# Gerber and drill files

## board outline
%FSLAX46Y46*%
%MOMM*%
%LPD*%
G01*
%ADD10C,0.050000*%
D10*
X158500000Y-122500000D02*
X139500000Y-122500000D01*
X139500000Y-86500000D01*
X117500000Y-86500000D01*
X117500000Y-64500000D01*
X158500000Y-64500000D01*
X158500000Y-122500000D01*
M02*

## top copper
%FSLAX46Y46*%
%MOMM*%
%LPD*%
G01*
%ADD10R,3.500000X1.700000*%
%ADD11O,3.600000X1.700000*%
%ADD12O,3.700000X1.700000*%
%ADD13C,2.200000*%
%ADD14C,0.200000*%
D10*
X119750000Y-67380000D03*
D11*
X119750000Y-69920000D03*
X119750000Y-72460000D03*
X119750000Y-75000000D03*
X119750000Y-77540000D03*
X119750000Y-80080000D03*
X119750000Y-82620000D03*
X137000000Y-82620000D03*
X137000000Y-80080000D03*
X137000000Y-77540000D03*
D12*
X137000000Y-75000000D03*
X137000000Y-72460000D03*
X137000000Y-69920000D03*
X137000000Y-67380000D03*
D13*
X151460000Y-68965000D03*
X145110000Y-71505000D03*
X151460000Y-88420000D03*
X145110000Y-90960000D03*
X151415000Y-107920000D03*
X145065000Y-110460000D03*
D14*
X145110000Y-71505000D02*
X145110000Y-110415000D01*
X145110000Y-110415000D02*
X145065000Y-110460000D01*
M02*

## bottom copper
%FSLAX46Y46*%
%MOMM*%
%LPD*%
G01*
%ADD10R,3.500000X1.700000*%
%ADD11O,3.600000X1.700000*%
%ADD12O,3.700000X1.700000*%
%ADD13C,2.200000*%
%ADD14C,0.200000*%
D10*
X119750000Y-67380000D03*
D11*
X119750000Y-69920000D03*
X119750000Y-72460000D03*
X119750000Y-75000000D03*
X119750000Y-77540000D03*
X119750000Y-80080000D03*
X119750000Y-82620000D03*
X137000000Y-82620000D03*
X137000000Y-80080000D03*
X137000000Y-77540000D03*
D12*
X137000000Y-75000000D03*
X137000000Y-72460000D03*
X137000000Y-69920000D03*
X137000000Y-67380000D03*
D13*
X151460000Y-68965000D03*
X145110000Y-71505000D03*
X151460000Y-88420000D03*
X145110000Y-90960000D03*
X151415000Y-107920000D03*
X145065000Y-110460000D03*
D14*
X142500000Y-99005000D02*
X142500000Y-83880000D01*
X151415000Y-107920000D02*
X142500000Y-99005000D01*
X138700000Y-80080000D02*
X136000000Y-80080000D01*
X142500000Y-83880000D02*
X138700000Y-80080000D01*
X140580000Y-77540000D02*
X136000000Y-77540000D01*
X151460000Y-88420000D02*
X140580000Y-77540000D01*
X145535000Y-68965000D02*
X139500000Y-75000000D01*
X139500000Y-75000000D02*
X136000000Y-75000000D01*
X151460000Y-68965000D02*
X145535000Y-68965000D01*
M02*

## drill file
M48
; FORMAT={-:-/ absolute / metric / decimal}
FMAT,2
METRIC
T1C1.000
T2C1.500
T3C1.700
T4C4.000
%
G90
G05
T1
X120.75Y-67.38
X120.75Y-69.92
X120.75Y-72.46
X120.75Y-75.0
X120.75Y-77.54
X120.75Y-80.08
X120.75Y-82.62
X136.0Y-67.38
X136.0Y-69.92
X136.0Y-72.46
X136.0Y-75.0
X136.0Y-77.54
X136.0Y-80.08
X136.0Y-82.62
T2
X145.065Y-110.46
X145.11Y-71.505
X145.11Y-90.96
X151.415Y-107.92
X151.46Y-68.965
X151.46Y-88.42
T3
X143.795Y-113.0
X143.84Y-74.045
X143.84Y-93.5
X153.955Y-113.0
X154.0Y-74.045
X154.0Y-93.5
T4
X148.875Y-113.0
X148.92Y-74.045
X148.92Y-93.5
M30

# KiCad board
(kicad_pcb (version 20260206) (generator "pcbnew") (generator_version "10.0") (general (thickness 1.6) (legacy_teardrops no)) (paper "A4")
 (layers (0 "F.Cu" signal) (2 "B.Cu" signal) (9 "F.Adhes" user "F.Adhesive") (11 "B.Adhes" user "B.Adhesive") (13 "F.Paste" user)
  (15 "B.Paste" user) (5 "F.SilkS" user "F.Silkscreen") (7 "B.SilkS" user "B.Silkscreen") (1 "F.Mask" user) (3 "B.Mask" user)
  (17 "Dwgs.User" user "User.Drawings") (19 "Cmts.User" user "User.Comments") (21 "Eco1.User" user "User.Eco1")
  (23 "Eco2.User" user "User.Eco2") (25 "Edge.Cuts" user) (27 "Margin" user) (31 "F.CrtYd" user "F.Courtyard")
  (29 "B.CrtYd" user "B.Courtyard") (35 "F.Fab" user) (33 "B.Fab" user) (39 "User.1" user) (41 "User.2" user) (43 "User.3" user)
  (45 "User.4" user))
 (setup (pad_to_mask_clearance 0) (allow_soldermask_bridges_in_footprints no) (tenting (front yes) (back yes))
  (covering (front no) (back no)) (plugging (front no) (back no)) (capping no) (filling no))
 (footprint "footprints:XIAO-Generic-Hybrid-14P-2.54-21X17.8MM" (layer "F.Cu") (at 128.375 75)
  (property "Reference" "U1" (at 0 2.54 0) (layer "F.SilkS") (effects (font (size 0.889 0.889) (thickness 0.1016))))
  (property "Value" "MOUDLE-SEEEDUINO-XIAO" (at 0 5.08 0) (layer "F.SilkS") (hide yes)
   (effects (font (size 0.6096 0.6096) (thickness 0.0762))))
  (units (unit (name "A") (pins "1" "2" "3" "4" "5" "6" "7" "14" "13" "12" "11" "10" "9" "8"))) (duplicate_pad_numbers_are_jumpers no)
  (pad "1" thru_hole rect (at -7.625 -7.62) (size 3.5 1.7) (drill 1 (offset -1 0)) (layers "*.Cu" "*.Mask") (remove_unused_layers no)
   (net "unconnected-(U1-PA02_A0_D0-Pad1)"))
  (pad "2" thru_hole oval (at -7.625 -5.08) (size 3.6 1.7) (drill 1 (offset -1 0)) (layers "*.Cu" "*.Mask") (remove_unused_layers no)
   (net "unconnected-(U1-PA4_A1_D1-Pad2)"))
  (pad "3" thru_hole oval (at -7.625 -2.54) (size 3.6 1.7) (drill 1 (offset -1 0)) (layers "*.Cu" "*.Mask") (remove_unused_layers no)
   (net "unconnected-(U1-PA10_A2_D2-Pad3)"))
  (pad "4" thru_hole oval (at -7.625 0) (size 3.6 1.7) (drill 1 (offset -1 0)) (layers "*.Cu" "*.Mask") (remove_unused_layers no)
   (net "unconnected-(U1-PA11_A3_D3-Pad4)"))
  (pad "5" thru_hole oval (at -7.625 2.54) (size 3.6 1.7) (drill 1 (offset -1 0)) (layers "*.Cu" "*.Mask") (remove_unused_layers no)
   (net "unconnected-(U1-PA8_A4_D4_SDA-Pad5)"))
  (pad "6" thru_hole oval (at -7.625 5.08 180) (size 3.6 1.7) (drill 1 (offset 1 0)) (layers "*.Cu" "*.Mask") (remove_unused_layers no)
   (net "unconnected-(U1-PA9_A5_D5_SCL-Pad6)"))
  (pad "7" thru_hole oval (at -7.625 7.62) (size 3.6 1.7) (drill 1 (offset -1 0)) (layers "*.Cu" "*.Mask") (remove_unused_layers no)
   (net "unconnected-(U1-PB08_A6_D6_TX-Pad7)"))
  (pad "8" thru_hole oval (at 7.625 7.62) (size 3.6 1.7) (drill 1 (offset 1 0)) (layers "*.Cu" "*.Mask") (remove_unused_layers no)
   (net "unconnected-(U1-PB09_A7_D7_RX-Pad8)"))
  (pad "9" thru_hole oval (at 7.625 5.08) (size 3.6 1.7) (drill 1 (offset 1 0)) (layers "*.Cu" "*.Mask") (remove_unused_layers no)
   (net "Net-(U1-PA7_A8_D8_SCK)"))
  (pad "10" thru_hole oval (at 7.625 2.54) (size 3.6 1.7) (drill 1 (offset 1 0)) (layers "*.Cu" "*.Mask") (remove_unused_layers no)
   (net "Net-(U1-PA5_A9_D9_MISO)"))
  (pad "11" thru_hole oval (at 7.625 0) (size 3.7 1.7) (drill 1 (offset 1 0)) (layers "*.Cu" "*.Mask") (remove_unused_layers no)
   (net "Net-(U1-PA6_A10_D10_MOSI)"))
  (pad "12" thru_hole oval (at 7.625 -2.54) (size 3.7 1.7) (drill 1 (offset 1 0)) (layers "*.Cu" "*.Mask") (remove_unused_layers no)
   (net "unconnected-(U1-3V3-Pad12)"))
  (pad "13" thru_hole oval (at 7.625 -5.08) (size 3.7 1.7) (drill 1 (offset 1 0)) (layers "*.Cu" "*.Mask") (remove_unused_layers no)
   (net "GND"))
  (pad "14" thru_hole oval (at 7.625 -7.62) (size 3.7 1.7) (drill 1 (offset 1 0)) (layers "*.Cu" "*.Mask") (remove_unused_layers no)
   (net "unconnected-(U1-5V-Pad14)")))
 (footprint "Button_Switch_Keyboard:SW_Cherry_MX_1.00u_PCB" (layer "F.Cu") (at 151.46 68.965)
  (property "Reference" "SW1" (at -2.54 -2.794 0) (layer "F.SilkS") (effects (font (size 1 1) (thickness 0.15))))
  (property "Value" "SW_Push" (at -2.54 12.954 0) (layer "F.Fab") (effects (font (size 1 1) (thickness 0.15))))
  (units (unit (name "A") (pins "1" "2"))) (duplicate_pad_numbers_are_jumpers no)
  (pad "" np_thru_hole circle (at -7.62 5.08) (size 1.7 1.7) (drill 1.7) (layers "*.Cu" "*.Mask"))
  (pad "" np_thru_hole circle (at -2.54 5.08) (size 4 4) (drill 4) (layers "*.Cu" "*.Mask"))
  (pad "" np_thru_hole circle (at 2.54 5.08) (size 1.7 1.7) (drill 1.7) (layers "*.Cu" "*.Mask"))
  (pad "1" thru_hole circle (at 0 0) (size 2.2 2.2) (drill 1.5) (layers "*.Cu" "*.Mask") (remove_unused_layers no)
   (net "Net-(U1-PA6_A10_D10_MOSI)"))
  (pad "2" thru_hole circle (at -6.35 2.54) (size 2.2 2.2) (drill 1.5) (layers "*.Cu" "*.Mask") (remove_unused_layers no) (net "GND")))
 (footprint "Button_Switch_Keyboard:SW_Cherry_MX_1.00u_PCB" (layer "F.Cu") (at 151.46 88.42)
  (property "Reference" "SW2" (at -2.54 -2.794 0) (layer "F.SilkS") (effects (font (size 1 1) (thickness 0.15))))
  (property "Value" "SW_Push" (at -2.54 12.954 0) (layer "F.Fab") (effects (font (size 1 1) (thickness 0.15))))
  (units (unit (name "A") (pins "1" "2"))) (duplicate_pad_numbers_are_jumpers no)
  (pad "" np_thru_hole circle (at -7.62 5.08) (size 1.7 1.7) (drill 1.7) (layers "*.Cu" "*.Mask"))
  (pad "" np_thru_hole circle (at -2.54 5.08) (size 4 4) (drill 4) (layers "*.Cu" "*.Mask"))
  (pad "" np_thru_hole circle (at 2.54 5.08) (size 1.7 1.7) (drill 1.7) (layers "*.Cu" "*.Mask"))
  (pad "1" thru_hole circle (at 0 0) (size 2.2 2.2) (drill 1.5) (layers "*.Cu" "*.Mask") (remove_unused_layers no)
   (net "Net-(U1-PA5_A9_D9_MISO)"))
  (pad "2" thru_hole circle (at -6.35 2.54) (size 2.2 2.2) (drill 1.5) (layers "*.Cu" "*.Mask") (remove_unused_layers no) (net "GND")))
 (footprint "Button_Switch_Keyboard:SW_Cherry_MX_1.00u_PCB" (layer "F.Cu") (at 151.415 107.92)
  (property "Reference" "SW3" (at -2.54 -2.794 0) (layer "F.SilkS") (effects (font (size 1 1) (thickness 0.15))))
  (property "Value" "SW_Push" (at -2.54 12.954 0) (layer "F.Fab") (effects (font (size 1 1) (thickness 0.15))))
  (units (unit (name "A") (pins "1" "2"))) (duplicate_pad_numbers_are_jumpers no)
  (pad "" np_thru_hole circle (at -7.62 5.08) (size 1.7 1.7) (drill 1.7) (layers "*.Cu" "*.Mask"))
  (pad "" np_thru_hole circle (at -2.54 5.08) (size 4 4) (drill 4) (layers "*.Cu" "*.Mask"))
  (pad "" np_thru_hole circle (at 2.54 5.08) (size 1.7 1.7) (drill 1.7) (layers "*.Cu" "*.Mask"))
  (pad "1" thru_hole circle (at 0 0) (size 2.2 2.2) (drill 1.5) (layers "*.Cu" "*.Mask") (remove_unused_layers no)
   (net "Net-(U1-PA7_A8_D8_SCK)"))
  (pad "2" thru_hole circle (at -6.35 2.54) (size 2.2 2.2) (drill 1.5) (layers "*.Cu" "*.Mask") (remove_unused_layers no) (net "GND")))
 (gr_poly
  (pts (xy 158.5 122.5) (xy 139.5 122.5) (xy 139.5 86.5) (xy 117.5 86.5) (xy 117.5 64.5) (xy 158.5 64.5)) (stroke (width 0.05) (type solid))
  (fill no) (layer "Edge.Cuts"))
 (segment (start 142.5 99.005) (end 142.5 83.88) (width 0.2) (layer "B.Cu") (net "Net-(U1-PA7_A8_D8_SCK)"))
 (segment (start 151.415 107.92) (end 142.5 99.005) (width 0.2) (layer "B.Cu") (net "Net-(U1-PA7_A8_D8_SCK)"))
 (segment (start 138.7 80.08) (end 136 80.08) (width 0.2) (layer "B.Cu") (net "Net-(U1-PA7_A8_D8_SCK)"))
 (segment (start 142.5 83.88) (end 138.7 80.08) (width 0.2) (layer "B.Cu") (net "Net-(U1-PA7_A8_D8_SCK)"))
 (segment (start 140.58 77.54) (end 136 77.54) (width 0.2) (layer "B.Cu") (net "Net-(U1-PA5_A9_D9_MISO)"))
 (segment (start 151.46 88.42) (end 140.58 77.54) (width 0.2) (layer "B.Cu") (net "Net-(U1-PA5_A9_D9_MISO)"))
 (segment (start 145.535 68.965) (end 139.5 75) (width 0.2) (layer "B.Cu") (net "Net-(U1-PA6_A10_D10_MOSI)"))
 (segment (start 139.5 75) (end 136 75) (width 0.2) (layer "B.Cu") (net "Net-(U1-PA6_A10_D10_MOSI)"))
 (segment (start 151.46 68.965) (end 145.535 68.965) (width 0.2) (layer "B.Cu") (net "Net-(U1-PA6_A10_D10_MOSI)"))
 (segment (start 145.11 71.505) (end 145.11 110.415) (width 0.2) (layer "F.Cu") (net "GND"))
 (segment (start 145.11 110.415) (end 145.065 110.46) (width 0.2) (layer "F.Cu") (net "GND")))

